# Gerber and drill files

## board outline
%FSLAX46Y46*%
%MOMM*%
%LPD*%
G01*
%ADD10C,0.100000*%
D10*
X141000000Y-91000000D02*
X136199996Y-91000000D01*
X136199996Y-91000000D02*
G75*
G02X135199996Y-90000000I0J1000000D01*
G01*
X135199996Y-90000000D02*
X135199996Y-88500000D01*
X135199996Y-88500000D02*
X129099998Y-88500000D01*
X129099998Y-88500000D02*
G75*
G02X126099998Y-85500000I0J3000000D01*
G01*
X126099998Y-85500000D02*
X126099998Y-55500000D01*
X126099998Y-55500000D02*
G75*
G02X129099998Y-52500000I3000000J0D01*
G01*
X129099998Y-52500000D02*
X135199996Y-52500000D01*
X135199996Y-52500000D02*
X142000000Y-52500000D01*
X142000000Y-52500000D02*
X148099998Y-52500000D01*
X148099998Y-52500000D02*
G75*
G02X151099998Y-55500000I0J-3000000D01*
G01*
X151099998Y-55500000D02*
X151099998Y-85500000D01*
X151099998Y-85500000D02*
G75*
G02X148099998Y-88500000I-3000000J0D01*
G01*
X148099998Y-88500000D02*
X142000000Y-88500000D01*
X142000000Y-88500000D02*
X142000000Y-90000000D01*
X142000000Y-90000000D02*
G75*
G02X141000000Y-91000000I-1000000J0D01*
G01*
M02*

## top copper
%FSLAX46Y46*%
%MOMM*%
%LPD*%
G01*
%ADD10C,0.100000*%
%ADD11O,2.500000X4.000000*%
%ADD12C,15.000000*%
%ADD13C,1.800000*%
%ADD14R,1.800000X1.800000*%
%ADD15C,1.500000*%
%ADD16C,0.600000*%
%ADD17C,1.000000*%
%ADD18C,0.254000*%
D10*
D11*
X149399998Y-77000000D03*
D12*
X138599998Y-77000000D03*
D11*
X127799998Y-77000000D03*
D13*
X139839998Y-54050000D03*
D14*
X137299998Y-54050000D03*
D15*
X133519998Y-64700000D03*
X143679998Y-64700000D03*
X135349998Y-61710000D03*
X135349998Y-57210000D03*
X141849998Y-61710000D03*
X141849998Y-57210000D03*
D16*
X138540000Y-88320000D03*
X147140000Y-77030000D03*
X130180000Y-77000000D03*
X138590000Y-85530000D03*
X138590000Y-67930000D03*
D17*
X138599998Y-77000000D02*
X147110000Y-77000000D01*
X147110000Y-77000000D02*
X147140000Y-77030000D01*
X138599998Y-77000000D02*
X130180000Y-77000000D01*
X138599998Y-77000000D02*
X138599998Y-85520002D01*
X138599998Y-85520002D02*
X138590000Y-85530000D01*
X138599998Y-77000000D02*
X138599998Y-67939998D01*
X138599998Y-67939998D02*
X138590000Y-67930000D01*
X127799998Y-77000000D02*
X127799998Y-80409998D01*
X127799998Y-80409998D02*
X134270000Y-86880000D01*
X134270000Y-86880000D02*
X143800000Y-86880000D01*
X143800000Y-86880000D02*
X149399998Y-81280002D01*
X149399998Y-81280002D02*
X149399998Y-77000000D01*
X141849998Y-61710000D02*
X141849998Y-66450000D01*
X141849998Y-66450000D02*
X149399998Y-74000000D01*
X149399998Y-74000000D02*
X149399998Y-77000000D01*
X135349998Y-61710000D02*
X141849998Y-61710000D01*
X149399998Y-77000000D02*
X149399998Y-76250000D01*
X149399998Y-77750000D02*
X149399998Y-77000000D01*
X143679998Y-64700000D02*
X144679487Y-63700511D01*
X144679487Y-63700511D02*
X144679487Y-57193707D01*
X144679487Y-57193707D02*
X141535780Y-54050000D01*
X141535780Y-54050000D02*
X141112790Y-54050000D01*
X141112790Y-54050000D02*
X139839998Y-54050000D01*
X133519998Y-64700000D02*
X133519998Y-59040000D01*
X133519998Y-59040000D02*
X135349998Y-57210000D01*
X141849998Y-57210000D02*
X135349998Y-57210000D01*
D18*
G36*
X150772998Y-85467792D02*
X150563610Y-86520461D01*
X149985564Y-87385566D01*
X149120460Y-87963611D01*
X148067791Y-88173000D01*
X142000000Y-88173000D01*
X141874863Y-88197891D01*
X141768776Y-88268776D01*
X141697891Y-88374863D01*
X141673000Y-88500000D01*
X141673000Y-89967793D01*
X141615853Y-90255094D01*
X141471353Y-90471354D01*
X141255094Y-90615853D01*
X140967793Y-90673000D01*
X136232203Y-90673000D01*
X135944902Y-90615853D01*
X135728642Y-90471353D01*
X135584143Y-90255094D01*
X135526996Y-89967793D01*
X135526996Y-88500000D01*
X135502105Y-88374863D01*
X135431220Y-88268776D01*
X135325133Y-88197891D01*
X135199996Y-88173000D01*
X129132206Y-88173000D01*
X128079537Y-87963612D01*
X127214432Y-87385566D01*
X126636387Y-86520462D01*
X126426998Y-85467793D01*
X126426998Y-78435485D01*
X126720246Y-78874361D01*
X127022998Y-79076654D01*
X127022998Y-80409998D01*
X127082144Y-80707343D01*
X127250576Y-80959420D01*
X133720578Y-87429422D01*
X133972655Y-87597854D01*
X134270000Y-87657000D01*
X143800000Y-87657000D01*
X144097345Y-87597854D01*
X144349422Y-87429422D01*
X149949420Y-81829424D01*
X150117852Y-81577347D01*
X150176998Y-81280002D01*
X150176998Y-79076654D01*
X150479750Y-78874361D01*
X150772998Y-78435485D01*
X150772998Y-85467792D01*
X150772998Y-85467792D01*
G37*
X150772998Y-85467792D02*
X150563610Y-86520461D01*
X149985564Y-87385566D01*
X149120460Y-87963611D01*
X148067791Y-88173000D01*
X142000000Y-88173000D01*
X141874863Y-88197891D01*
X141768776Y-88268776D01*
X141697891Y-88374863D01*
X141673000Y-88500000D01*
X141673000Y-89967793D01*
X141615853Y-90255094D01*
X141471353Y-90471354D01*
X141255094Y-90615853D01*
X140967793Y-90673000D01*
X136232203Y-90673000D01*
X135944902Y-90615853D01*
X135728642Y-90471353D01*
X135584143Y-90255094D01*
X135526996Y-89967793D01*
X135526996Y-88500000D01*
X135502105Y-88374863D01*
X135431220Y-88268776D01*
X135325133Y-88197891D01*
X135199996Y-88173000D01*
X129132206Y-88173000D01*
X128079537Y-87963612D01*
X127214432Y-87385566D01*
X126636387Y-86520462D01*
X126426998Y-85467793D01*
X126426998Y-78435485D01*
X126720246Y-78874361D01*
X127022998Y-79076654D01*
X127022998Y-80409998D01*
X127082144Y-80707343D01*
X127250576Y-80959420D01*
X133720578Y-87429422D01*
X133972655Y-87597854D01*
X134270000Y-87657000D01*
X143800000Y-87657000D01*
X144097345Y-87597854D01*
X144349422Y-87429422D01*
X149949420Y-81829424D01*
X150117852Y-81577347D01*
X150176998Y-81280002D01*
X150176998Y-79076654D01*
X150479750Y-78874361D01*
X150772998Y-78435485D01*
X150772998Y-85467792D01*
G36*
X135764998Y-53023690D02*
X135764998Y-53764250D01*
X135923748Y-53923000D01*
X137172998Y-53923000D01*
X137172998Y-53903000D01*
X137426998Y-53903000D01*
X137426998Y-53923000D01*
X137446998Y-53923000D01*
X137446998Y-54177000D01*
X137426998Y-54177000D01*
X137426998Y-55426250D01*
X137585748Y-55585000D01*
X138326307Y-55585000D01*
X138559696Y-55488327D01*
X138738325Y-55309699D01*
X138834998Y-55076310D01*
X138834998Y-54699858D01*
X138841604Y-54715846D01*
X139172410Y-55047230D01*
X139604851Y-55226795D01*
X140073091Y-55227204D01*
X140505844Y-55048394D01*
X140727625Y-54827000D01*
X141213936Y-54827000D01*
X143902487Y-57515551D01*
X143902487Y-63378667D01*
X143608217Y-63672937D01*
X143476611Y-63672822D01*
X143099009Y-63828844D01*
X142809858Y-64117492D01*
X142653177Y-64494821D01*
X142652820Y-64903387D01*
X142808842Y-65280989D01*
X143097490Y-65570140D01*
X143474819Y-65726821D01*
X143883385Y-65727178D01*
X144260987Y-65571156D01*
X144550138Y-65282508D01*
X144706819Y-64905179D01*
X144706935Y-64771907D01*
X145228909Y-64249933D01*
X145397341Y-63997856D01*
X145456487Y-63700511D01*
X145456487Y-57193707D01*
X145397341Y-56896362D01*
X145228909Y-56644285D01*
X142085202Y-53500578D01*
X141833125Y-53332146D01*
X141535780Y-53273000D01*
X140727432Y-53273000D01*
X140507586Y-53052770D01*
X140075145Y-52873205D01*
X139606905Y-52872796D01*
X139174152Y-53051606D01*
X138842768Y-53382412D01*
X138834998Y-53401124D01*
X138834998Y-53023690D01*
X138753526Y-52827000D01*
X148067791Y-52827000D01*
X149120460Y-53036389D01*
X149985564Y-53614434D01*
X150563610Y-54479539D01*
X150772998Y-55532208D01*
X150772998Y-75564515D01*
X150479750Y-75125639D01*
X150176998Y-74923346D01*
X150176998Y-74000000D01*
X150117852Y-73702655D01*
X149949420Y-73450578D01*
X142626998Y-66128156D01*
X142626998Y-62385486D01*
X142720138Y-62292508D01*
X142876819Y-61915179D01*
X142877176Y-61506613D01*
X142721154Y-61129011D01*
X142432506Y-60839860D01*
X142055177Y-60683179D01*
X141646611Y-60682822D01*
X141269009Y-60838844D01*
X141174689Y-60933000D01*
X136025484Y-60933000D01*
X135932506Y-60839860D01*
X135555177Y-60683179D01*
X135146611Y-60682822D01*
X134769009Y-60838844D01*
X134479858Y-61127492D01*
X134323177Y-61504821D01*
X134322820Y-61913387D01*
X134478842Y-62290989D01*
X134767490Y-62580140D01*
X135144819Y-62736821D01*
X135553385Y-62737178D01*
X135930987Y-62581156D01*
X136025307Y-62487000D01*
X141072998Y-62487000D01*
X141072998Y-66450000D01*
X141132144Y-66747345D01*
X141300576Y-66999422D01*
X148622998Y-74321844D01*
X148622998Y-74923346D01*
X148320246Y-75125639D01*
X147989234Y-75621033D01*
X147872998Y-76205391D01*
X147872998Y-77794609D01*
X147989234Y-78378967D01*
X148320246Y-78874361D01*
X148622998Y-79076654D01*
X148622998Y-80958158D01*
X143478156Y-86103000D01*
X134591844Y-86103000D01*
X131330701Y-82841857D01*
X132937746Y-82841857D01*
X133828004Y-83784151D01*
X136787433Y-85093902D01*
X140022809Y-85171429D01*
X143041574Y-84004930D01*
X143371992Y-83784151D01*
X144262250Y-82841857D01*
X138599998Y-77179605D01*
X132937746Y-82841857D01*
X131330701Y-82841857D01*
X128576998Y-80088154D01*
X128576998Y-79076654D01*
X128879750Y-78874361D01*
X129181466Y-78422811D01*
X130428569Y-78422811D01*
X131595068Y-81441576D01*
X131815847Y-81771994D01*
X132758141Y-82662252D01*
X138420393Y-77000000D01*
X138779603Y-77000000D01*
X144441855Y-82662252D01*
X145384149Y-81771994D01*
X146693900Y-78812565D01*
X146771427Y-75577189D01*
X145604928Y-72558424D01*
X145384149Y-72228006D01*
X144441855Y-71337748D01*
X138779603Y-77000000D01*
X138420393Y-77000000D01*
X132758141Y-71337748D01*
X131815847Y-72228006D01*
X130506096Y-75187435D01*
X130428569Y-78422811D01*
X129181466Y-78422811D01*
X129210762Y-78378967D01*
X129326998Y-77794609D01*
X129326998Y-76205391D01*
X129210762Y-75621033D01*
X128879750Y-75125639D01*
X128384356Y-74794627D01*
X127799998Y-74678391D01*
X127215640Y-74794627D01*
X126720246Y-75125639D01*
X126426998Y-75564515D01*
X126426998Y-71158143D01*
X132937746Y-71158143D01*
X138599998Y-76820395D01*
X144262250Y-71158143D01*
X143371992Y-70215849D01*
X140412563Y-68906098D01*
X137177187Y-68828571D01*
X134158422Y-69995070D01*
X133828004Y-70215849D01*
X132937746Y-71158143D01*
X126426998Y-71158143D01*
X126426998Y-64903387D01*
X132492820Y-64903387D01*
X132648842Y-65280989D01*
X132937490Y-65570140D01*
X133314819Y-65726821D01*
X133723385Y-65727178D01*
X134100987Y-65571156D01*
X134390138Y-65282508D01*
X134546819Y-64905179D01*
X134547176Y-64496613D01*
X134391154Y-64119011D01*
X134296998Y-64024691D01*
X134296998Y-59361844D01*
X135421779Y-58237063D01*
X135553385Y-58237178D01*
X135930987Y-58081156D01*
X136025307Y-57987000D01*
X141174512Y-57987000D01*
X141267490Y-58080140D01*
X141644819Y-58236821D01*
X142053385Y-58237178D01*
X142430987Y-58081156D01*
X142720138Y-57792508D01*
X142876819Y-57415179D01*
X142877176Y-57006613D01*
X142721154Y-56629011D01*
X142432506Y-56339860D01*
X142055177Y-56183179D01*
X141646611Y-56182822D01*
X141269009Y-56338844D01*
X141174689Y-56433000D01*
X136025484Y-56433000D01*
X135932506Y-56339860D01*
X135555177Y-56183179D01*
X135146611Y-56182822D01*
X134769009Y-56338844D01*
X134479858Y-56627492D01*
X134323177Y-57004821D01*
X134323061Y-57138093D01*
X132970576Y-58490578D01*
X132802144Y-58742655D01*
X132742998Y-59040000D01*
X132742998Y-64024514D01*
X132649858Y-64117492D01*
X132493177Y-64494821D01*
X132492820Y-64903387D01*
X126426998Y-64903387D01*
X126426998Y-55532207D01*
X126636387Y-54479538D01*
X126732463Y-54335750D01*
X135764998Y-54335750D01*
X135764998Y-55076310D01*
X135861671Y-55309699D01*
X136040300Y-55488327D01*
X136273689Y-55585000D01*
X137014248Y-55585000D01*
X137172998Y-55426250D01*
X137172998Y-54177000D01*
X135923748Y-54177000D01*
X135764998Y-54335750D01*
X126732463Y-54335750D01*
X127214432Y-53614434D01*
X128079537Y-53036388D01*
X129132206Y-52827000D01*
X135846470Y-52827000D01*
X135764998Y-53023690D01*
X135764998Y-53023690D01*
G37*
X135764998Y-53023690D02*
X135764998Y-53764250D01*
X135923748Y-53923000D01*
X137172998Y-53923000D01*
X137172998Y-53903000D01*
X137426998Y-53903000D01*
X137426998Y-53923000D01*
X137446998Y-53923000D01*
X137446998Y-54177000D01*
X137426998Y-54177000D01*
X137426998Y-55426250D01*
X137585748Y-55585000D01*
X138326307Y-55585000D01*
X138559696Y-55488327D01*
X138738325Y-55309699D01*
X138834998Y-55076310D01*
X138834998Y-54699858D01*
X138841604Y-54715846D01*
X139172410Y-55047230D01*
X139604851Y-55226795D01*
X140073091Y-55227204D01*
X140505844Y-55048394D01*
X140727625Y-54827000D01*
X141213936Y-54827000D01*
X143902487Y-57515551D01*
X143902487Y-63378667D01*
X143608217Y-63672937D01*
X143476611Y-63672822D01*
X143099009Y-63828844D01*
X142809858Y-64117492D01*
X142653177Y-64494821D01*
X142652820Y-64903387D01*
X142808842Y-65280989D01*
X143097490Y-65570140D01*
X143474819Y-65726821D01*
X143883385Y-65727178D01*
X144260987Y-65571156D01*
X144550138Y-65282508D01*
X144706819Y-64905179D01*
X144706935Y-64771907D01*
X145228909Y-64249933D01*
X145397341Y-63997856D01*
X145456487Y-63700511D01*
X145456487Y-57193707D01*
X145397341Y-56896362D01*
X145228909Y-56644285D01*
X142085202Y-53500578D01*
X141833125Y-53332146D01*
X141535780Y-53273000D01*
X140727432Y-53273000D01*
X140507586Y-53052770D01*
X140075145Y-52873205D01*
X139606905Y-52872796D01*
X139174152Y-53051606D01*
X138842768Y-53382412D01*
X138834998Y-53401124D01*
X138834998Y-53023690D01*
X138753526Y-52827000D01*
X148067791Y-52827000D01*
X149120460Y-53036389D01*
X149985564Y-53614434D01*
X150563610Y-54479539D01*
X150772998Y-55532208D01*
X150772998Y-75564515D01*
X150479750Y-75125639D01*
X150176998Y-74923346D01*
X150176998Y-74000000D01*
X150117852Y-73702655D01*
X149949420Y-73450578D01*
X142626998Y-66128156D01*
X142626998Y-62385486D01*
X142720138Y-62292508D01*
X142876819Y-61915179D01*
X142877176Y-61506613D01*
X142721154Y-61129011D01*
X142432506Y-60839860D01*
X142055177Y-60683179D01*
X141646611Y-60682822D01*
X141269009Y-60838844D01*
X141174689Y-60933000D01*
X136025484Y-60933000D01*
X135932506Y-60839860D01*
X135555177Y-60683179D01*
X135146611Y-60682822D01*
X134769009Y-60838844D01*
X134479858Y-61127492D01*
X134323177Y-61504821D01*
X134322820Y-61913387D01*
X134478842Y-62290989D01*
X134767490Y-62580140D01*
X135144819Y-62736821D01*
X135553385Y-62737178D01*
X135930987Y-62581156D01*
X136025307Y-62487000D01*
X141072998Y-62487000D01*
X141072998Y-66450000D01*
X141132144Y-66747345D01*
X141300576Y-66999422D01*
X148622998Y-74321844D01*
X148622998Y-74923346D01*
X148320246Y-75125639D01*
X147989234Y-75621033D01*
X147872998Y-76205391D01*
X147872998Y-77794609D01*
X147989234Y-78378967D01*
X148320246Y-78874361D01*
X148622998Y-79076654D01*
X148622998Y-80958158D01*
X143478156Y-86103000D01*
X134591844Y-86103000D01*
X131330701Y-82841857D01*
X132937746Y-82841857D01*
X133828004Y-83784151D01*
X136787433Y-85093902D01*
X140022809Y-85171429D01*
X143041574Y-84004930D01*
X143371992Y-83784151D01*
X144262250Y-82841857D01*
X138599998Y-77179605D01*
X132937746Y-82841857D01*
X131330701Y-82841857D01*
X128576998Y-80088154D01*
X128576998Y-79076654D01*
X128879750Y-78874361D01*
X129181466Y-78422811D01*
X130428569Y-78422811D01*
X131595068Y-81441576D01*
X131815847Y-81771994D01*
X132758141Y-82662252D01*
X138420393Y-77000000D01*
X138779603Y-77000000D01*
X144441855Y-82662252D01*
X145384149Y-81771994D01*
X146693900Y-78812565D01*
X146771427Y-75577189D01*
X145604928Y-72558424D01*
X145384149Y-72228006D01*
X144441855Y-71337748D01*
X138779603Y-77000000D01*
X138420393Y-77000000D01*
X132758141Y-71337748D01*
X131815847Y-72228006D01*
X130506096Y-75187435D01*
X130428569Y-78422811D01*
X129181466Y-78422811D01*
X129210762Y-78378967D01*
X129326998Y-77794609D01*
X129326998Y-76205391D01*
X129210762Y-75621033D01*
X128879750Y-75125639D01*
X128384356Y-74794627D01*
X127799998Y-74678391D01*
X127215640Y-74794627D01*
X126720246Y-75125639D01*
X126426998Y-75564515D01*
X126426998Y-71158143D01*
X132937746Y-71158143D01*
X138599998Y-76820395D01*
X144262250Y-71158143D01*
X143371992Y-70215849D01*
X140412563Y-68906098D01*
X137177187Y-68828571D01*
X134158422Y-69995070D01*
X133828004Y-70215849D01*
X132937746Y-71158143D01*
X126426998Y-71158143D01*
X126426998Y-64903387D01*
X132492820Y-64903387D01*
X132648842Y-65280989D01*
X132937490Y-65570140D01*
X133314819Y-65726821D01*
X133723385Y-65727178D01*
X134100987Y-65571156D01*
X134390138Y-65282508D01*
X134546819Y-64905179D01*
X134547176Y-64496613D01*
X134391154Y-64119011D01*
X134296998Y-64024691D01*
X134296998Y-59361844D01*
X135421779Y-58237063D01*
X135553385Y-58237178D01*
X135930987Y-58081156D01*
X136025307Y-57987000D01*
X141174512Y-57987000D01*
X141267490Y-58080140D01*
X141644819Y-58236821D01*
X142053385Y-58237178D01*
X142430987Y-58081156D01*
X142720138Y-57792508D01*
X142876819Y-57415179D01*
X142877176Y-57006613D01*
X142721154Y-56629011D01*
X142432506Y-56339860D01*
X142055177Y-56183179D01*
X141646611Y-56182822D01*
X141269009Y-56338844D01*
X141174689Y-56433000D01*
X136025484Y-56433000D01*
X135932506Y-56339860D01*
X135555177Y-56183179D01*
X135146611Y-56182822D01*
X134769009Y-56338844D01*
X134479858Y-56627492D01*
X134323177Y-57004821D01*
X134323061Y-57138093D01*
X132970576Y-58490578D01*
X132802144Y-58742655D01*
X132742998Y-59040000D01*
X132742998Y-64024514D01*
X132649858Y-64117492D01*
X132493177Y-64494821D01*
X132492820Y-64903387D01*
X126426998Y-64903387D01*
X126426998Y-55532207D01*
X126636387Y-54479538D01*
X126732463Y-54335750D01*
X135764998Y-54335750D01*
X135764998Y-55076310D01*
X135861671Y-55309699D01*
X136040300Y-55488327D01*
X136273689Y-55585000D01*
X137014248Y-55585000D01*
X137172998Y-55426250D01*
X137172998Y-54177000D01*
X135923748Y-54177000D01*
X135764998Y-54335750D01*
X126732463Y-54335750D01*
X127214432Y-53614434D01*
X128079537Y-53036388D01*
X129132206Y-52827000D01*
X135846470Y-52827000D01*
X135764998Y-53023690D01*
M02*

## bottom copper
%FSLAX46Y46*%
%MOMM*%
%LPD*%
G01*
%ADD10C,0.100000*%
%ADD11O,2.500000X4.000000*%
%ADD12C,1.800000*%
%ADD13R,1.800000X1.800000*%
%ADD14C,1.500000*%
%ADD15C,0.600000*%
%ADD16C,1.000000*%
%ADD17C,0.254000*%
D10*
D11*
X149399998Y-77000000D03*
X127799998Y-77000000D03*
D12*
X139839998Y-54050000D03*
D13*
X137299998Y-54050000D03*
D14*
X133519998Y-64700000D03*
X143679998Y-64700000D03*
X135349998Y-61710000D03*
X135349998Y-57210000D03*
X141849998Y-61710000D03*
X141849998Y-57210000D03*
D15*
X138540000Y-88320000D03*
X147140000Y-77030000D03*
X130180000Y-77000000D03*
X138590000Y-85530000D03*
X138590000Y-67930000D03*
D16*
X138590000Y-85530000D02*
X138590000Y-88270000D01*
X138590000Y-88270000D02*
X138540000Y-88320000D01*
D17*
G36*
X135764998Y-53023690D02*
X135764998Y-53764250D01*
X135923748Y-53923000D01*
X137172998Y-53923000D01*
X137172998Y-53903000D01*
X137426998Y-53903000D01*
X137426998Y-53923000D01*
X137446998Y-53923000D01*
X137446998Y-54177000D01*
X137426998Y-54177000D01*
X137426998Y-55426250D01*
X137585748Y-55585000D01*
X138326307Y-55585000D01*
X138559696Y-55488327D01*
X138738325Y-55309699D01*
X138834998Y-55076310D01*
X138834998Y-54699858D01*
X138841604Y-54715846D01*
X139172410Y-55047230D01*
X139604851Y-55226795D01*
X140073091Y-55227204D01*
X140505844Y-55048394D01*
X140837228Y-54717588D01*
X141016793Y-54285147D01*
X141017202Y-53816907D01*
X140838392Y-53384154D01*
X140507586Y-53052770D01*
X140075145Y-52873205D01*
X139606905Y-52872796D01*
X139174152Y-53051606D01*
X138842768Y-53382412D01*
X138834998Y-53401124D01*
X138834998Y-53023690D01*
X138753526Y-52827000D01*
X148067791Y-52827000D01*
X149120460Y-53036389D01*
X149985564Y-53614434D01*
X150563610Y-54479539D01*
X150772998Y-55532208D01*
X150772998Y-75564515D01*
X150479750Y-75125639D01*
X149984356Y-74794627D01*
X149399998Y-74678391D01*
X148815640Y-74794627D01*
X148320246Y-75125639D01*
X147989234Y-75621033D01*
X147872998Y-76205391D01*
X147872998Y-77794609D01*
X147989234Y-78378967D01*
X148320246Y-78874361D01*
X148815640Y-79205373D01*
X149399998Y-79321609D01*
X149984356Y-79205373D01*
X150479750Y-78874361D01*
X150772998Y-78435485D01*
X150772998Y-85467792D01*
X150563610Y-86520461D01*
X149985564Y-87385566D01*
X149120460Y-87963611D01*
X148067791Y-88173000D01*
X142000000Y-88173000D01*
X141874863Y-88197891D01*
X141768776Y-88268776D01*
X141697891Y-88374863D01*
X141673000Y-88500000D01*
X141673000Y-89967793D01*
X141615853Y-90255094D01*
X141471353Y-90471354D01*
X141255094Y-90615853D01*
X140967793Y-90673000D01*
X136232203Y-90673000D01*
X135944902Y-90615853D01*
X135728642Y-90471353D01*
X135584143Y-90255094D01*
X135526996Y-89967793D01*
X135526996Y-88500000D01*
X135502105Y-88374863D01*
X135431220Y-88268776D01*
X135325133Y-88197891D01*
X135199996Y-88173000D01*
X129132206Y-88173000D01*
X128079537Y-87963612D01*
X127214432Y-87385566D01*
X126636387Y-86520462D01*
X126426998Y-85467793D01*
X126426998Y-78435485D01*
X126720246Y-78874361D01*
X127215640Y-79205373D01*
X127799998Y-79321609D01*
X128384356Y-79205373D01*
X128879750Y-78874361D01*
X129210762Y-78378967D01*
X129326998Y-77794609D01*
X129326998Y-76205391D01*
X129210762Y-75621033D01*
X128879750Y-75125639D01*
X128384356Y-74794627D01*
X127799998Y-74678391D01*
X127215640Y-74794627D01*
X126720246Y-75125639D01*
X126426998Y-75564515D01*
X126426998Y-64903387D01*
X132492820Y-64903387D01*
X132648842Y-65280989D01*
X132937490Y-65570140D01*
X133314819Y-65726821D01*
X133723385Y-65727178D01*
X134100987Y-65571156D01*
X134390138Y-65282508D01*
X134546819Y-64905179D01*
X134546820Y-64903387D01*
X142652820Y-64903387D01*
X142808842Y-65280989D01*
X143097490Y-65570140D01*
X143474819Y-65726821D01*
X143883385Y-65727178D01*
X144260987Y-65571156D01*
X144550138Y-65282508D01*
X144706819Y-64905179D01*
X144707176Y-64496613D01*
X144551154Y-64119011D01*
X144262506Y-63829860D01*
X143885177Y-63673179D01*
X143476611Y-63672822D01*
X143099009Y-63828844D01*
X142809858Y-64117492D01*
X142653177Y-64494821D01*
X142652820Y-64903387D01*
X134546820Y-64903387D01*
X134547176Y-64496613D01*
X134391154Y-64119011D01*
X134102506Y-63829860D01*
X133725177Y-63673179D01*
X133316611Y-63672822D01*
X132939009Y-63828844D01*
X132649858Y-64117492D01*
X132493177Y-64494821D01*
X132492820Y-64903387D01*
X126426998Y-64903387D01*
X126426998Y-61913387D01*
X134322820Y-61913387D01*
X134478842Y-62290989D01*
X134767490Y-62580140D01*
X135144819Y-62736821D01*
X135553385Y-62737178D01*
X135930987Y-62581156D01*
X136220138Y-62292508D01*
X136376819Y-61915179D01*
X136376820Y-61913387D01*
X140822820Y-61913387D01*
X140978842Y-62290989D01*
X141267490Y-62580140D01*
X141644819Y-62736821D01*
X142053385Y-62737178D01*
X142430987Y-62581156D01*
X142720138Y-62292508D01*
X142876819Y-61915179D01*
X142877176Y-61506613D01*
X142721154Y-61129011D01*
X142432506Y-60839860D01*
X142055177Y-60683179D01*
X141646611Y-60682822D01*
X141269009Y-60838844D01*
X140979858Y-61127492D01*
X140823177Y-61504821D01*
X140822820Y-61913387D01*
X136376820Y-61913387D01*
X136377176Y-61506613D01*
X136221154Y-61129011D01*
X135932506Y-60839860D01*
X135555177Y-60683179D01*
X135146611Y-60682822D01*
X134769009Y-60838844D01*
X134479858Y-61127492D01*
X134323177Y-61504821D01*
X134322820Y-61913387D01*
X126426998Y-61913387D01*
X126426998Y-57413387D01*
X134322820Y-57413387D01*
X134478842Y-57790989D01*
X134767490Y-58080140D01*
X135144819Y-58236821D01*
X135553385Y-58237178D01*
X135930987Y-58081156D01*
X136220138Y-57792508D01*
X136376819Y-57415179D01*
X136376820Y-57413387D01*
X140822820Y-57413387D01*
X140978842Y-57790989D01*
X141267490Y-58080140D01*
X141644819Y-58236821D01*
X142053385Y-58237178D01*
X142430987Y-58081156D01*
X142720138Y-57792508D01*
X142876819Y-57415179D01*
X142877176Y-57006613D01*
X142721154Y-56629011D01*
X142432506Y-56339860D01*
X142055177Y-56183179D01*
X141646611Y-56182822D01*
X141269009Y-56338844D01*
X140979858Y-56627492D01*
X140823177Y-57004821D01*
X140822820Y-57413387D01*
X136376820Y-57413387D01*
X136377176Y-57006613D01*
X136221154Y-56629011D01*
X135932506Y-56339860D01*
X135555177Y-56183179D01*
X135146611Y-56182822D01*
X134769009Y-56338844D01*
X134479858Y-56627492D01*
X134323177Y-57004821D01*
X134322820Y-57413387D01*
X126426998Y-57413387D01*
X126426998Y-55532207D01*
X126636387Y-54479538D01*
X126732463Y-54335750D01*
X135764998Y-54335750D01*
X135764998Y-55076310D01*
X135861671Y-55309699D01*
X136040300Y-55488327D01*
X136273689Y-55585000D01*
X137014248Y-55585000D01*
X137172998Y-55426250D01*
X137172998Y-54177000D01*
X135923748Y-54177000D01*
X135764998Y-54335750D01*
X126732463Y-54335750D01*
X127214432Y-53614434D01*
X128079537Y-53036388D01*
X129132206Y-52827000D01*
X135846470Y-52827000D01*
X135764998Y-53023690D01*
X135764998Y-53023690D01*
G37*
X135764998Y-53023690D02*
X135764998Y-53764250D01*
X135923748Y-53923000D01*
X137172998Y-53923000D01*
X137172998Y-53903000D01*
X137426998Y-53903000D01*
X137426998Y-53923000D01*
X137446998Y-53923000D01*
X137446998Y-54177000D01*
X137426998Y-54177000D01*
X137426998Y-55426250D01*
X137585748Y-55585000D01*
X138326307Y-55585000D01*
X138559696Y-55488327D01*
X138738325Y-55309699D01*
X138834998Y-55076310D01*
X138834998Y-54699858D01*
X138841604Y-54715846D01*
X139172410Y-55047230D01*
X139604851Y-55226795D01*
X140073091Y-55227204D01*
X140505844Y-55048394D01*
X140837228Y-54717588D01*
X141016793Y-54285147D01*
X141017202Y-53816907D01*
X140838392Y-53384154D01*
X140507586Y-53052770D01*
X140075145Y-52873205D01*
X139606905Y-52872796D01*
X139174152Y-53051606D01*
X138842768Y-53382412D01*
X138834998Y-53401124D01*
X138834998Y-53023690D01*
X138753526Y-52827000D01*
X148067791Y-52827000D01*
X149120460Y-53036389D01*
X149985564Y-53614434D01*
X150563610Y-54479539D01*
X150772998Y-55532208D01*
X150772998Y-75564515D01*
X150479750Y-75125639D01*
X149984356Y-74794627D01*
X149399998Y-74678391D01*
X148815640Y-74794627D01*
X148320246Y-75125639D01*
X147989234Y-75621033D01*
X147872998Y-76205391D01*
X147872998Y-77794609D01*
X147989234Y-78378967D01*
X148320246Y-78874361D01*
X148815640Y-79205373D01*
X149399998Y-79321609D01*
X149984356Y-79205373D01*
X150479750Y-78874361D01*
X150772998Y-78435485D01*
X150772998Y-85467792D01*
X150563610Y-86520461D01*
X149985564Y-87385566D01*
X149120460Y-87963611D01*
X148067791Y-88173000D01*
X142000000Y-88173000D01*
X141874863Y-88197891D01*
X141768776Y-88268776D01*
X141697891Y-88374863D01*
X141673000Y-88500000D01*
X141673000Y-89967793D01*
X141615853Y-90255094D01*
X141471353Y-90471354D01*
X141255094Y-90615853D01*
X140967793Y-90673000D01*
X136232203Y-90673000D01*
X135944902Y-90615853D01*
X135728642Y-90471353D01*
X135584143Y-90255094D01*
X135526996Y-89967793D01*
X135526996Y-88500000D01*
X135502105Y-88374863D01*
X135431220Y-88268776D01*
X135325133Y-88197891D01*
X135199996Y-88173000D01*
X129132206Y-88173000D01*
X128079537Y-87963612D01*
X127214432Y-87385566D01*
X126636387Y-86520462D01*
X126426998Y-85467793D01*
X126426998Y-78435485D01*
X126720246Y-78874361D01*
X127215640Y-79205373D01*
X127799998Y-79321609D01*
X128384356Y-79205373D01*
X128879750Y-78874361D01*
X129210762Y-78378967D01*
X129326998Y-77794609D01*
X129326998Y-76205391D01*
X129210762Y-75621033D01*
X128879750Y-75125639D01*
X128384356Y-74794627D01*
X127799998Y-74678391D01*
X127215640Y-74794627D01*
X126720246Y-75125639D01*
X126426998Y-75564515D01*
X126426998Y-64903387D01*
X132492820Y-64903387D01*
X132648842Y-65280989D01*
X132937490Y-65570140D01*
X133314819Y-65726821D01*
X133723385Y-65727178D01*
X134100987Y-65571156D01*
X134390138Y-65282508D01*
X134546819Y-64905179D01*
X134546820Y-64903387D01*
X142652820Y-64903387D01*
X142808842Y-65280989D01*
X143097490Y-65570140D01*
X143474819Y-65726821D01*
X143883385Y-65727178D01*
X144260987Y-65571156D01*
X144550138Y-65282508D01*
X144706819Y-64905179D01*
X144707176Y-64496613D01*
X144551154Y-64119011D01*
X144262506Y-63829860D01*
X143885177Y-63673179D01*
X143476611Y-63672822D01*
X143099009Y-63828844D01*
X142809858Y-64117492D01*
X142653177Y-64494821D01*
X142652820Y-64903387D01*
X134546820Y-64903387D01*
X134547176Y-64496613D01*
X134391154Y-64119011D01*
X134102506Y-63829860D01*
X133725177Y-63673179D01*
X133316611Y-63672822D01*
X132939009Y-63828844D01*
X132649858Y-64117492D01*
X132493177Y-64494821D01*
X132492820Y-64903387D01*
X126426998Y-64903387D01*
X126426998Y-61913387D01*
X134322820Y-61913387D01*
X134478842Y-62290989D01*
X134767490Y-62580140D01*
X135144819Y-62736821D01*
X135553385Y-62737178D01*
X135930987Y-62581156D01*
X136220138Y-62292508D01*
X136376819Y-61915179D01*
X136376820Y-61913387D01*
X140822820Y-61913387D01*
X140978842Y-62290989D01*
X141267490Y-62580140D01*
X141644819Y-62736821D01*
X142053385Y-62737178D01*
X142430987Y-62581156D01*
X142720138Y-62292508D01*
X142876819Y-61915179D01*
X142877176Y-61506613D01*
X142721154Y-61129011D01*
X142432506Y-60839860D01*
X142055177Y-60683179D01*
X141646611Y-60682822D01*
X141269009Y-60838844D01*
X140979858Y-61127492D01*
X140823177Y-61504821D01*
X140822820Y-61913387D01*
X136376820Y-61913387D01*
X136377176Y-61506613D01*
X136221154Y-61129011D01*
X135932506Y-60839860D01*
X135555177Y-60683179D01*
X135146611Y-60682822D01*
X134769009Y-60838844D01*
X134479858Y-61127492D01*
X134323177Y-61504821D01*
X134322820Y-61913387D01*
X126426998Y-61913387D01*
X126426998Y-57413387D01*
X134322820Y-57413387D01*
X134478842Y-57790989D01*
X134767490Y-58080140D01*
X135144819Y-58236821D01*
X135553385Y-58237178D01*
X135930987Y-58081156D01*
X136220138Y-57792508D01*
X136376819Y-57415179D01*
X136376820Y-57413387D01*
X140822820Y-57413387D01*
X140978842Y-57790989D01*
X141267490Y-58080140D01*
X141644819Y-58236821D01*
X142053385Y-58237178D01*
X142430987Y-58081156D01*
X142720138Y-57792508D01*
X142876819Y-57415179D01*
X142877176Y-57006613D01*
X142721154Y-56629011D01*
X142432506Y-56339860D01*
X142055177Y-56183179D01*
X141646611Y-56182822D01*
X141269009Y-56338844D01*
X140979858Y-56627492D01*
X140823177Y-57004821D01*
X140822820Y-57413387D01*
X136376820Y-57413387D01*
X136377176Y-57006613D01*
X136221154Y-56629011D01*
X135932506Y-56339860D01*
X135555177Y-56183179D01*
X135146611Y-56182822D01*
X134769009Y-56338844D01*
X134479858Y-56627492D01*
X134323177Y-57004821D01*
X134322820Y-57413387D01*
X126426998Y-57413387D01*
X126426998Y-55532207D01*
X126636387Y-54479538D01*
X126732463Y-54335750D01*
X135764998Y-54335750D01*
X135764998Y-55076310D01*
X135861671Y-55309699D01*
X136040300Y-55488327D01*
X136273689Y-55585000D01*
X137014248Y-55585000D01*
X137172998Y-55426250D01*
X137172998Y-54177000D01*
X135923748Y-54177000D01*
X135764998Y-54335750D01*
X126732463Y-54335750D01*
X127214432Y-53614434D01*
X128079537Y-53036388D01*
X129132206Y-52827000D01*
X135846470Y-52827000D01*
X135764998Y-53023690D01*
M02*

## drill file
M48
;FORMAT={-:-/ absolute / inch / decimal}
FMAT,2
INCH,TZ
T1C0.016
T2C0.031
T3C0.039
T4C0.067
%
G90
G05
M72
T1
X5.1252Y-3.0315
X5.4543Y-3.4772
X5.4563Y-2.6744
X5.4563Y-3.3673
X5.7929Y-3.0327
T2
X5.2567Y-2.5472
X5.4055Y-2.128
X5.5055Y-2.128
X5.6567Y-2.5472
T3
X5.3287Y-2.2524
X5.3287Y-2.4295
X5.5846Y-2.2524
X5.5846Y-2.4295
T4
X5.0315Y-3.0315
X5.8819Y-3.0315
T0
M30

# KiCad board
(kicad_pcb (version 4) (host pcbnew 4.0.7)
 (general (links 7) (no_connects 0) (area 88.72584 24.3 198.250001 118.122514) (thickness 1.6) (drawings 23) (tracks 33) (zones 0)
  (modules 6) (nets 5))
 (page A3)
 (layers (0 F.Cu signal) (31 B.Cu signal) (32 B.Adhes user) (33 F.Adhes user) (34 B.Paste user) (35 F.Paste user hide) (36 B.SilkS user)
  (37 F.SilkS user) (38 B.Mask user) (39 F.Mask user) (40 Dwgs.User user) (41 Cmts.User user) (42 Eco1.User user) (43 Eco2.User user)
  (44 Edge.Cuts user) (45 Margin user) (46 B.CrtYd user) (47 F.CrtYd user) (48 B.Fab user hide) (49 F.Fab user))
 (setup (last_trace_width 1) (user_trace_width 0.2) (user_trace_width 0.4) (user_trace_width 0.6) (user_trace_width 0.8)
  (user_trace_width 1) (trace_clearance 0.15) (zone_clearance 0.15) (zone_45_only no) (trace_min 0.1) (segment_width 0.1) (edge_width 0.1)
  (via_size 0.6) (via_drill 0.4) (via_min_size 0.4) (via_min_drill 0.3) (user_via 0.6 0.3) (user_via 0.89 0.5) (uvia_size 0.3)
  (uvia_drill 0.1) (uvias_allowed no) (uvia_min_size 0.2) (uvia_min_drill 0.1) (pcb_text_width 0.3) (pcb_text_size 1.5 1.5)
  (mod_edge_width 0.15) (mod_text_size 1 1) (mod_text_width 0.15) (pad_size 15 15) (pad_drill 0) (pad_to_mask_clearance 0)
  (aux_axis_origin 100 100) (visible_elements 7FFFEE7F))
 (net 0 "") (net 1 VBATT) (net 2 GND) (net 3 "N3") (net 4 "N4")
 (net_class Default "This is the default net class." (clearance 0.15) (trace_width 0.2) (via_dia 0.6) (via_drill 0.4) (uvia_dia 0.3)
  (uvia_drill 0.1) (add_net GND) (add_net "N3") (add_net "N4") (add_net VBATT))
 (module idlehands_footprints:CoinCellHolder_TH (layer F.Cu) (at 138.599998 77 180)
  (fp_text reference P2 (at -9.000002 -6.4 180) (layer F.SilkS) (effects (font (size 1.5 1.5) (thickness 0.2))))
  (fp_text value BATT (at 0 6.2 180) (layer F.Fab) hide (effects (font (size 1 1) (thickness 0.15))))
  (pad 2 thru_hole oval (at -10.8 0 180) (size 2.5 4) (drill 1.7) (layers *.Cu *.Mask F.SilkS) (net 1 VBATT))
  (pad 1 smd circle (at 0 0 180) (size 15 15) (layers F.Cu F.Paste F.Mask) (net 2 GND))
  (pad 2 thru_hole oval (at 10.8 0 180) (size 2.5 4) (drill 1.7) (layers *.Cu *.Mask F.SilkS) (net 1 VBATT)))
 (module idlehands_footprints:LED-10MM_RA (layer F.Cu) (at 138.599998 54)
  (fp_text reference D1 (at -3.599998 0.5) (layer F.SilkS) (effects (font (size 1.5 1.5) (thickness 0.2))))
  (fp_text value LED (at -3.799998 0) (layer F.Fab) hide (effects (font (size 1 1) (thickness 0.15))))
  (pad 2 thru_hole circle (at 1.24 0.05 180) (size 1.8 1.8) (drill 0.8) (layers *.Cu *.Mask F.SilkS) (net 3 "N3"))
  (pad 1 thru_hole rect (at -1.3 0.05 180) (size 1.8 1.8) (drill 0.8) (layers *.Cu *.Mask F.SilkS) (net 2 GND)))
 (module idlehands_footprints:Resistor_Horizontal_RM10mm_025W (layer F.Cu) (at 138.599998 64.7)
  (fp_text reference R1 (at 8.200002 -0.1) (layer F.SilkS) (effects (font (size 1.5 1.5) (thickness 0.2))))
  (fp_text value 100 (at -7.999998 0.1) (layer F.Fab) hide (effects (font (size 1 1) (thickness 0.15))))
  (pad 1 thru_hole circle (at -5.08 0) (size 1.5 1.5) (drill 0.8) (layers *.Cu *.SilkS *.Mask) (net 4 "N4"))
  (pad 2 thru_hole circle (at 5.08 0) (size 1.5 1.5) (drill 0.8) (layers *.Cu *.SilkS *.Mask) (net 3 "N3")))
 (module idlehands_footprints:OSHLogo (layer B.Cu) (at 132.2 84.8 90)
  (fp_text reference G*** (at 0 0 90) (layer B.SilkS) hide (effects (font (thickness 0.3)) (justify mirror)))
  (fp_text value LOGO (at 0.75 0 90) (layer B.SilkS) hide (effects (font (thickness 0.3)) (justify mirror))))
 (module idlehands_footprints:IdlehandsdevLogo (layer B.Cu) (at 132 78.6 270)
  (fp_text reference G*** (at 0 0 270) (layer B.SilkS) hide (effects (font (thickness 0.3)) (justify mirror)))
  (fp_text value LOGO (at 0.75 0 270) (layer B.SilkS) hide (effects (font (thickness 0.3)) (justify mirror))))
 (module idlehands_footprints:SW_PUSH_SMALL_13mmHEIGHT (layer F.Cu) (at 138.599998 59.46 180)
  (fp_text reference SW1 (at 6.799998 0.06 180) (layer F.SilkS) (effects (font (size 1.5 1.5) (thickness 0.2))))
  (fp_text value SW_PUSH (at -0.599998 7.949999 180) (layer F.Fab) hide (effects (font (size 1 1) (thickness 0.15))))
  (pad 1 thru_hole circle (at 3.25 -2.25 180) (size 1.5 1.5) (drill 0.99) (layers *.Cu *.Mask F.SilkS) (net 1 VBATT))
  (pad 2 thru_hole circle (at 3.25 2.25 180) (size 1.5 1.5) (drill 0.99) (layers *.Cu *.Mask F.SilkS) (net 4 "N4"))
  (pad 1 thru_hole circle (at -3.25 -2.25 180) (size 1.5 1.5) (drill 0.99) (layers *.Cu *.Mask F.SilkS) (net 1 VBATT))
  (pad 2 thru_hole circle (at -3.25 2.25 180) (size 1.5 1.5) (drill 0.99) (layers *.Cu *.Mask F.SilkS) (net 4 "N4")))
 (gr_line (start 141 91) (end 136.199996 91) (layer Edge.Cuts) (width 0.1))
 (gr_arc (start 136.199996 90) (end 135.199996 90) (angle -90.000002) (layer Edge.Cuts) (width 0.1))
 (gr_line (start 135.199996 90) (end 135.199996 88.5) (layer Edge.Cuts) (width 0.1))
 (gr_line (start 135.199996 88.5) (end 129.099998 88.5) (layer Edge.Cuts) (width 0.1))
 (gr_arc (start 129.099998 85.5) (end 126.099998 85.5) (angle -90.000002) (layer Edge.Cuts) (width 0.1))
 (gr_line (start 126.099998 85.5) (end 126.099998 55.5) (layer Edge.Cuts) (width 0.1))
 (gr_arc (start 129.099998 55.5) (end 129.099998 52.5) (angle -90.000002) (layer Edge.Cuts) (width 0.1))
 (gr_line (start 129.099998 52.5) (end 135.199996 52.5) (layer Edge.Cuts) (width 0.1))
 (gr_line (start 135.199996 52.5) (end 142 52.5) (layer Edge.Cuts) (width 0.1))
 (gr_line (start 142 52.5) (end 148.099998 52.5) (layer Edge.Cuts) (width 0.1))
 (gr_arc (start 148.099998 55.5) (end 151.099998 55.5) (angle -90.000003) (layer Edge.Cuts) (width 0.1))
 (gr_line (start 151.099998 55.5) (end 151.099998 85.5) (layer Edge.Cuts) (width 0.1))
 (gr_arc (start 148.099998 85.5) (end 148.099998 88.5) (angle -90.000003) (layer Edge.Cuts) (width 0.1))
 (gr_line (start 148.099998 88.5) (end 142 88.5) (layer Edge.Cuts) (width 0.1))
 (gr_line (start 142 88.5) (end 142 90) (layer Edge.Cuts) (width 0.1))
 (gr_arc (start 141 90) (end 141 91) (angle -90.000003) (layer Edge.Cuts) (width 0.1))
 (segment (start 138.59 85.53) (end 138.59 88.27) (width 1) (layer B.Cu) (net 2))
 (segment (start 138.59 88.27) (end 138.54 88.32) (width 1) (layer B.Cu) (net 2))
 (via (at 138.54 88.32) (size 0.6) (drill 0.4) (layers F.Cu B.Cu) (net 2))
 (segment (start 138.599998 77) (end 147.11 77) (width 1) (layer F.Cu) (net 2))
 (segment (start 147.11 77) (end 147.14 77.03) (width 1) (layer F.Cu) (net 2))
 (via (at 147.14 77.03) (size 0.6) (drill 0.4) (layers F.Cu B.Cu) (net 2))
 (segment (start 138.599998 77) (end 130.18 77) (width 1) (layer F.Cu) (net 2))
 (via (at 130.18 77) (size 0.6) (drill 0.4) (layers F.Cu B.Cu) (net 2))
 (segment (start 138.599998 77) (end 138.599998 85.520002) (width 1) (layer F.Cu) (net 2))
 (segment (start 138.599998 85.520002) (end 138.59 85.53) (width 1) (layer F.Cu) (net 2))
 (via (at 138.59 85.53) (size 0.6) (drill 0.4) (layers F.Cu B.Cu) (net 2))
 (segment (start 138.599998 77) (end 138.599998 67.939998) (width 1) (layer F.Cu) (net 2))
 (segment (start 138.599998 67.939998) (end 138.59 67.93) (width 1) (layer F.Cu) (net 2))
 (via (at 138.59 67.93) (size 0.6) (drill 0.4) (layers F.Cu B.Cu) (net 2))
 (segment (start 127.799998 77) (end 127.799998 80.409998) (width 1) (layer F.Cu) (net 1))
 (segment (start 127.799998 80.409998) (end 134.27 86.88) (width 1) (layer F.Cu) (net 1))
 (segment (start 134.27 86.88) (end 143.8 86.88) (width 1) (layer F.Cu) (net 1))
 (segment (start 143.8 86.88) (end 149.399998 81.280002) (width 1) (layer F.Cu) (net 1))
 (segment (start 149.399998 81.280002) (end 149.399998 77) (width 1) (layer F.Cu) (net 1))
 (segment (start 141.849998 61.71) (end 141.849998 66.45) (width 1) (layer F.Cu) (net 1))
 (segment (start 141.849998 66.45) (end 149.399998 74) (width 1) (layer F.Cu) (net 1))
 (segment (start 149.399998 74) (end 149.399998 77) (width 1) (layer F.Cu) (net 1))
 (segment (start 135.349998 61.71) (end 141.849998 61.71) (width 1) (layer F.Cu) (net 1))
 (segment (start 149.399998 77) (end 149.399998 76.25) (width 1) (layer F.Cu) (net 1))
 (segment (start 149.399998 77.75) (end 149.399998 77) (width 1) (layer F.Cu) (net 1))
 (segment (start 143.679998 64.7) (end 144.679487 63.700511) (width 1) (layer F.Cu) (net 3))
 (segment (start 144.679487 63.700511) (end 144.679487 57.193707) (width 1) (layer F.Cu) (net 3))
 (segment (start 144.679487 57.193707) (end 141.53578 54.05) (width 1) (layer F.Cu) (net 3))
 (segment (start 141.53578 54.05) (end 141.11279 54.05) (width 1) (layer F.Cu) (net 3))
 (segment (start 141.11279 54.05) (end 139.839998 54.05) (width 1) (layer F.Cu) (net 3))
 (segment (start 133.519998 64.7) (end 133.519998 59.04) (width 1) (layer F.Cu) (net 4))
 (segment (start 133.519998 59.04) (end 135.349998 57.21) (width 1) (layer F.Cu) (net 4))
 (segment (start 141.849998 57.21) (end 135.349998 57.21) (width 1) (layer F.Cu) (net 4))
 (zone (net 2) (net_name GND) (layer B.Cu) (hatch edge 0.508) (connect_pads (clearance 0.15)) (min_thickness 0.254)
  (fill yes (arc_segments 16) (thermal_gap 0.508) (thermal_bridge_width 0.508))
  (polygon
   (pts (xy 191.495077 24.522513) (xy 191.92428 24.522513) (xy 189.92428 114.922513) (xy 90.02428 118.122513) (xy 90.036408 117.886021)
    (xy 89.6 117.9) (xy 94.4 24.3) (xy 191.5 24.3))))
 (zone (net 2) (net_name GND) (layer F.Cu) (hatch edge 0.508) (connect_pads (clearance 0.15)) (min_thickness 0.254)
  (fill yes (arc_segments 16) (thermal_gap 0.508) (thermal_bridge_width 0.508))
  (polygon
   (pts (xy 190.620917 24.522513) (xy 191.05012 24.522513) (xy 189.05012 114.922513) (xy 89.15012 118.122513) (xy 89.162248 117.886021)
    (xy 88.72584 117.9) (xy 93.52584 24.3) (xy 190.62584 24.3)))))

